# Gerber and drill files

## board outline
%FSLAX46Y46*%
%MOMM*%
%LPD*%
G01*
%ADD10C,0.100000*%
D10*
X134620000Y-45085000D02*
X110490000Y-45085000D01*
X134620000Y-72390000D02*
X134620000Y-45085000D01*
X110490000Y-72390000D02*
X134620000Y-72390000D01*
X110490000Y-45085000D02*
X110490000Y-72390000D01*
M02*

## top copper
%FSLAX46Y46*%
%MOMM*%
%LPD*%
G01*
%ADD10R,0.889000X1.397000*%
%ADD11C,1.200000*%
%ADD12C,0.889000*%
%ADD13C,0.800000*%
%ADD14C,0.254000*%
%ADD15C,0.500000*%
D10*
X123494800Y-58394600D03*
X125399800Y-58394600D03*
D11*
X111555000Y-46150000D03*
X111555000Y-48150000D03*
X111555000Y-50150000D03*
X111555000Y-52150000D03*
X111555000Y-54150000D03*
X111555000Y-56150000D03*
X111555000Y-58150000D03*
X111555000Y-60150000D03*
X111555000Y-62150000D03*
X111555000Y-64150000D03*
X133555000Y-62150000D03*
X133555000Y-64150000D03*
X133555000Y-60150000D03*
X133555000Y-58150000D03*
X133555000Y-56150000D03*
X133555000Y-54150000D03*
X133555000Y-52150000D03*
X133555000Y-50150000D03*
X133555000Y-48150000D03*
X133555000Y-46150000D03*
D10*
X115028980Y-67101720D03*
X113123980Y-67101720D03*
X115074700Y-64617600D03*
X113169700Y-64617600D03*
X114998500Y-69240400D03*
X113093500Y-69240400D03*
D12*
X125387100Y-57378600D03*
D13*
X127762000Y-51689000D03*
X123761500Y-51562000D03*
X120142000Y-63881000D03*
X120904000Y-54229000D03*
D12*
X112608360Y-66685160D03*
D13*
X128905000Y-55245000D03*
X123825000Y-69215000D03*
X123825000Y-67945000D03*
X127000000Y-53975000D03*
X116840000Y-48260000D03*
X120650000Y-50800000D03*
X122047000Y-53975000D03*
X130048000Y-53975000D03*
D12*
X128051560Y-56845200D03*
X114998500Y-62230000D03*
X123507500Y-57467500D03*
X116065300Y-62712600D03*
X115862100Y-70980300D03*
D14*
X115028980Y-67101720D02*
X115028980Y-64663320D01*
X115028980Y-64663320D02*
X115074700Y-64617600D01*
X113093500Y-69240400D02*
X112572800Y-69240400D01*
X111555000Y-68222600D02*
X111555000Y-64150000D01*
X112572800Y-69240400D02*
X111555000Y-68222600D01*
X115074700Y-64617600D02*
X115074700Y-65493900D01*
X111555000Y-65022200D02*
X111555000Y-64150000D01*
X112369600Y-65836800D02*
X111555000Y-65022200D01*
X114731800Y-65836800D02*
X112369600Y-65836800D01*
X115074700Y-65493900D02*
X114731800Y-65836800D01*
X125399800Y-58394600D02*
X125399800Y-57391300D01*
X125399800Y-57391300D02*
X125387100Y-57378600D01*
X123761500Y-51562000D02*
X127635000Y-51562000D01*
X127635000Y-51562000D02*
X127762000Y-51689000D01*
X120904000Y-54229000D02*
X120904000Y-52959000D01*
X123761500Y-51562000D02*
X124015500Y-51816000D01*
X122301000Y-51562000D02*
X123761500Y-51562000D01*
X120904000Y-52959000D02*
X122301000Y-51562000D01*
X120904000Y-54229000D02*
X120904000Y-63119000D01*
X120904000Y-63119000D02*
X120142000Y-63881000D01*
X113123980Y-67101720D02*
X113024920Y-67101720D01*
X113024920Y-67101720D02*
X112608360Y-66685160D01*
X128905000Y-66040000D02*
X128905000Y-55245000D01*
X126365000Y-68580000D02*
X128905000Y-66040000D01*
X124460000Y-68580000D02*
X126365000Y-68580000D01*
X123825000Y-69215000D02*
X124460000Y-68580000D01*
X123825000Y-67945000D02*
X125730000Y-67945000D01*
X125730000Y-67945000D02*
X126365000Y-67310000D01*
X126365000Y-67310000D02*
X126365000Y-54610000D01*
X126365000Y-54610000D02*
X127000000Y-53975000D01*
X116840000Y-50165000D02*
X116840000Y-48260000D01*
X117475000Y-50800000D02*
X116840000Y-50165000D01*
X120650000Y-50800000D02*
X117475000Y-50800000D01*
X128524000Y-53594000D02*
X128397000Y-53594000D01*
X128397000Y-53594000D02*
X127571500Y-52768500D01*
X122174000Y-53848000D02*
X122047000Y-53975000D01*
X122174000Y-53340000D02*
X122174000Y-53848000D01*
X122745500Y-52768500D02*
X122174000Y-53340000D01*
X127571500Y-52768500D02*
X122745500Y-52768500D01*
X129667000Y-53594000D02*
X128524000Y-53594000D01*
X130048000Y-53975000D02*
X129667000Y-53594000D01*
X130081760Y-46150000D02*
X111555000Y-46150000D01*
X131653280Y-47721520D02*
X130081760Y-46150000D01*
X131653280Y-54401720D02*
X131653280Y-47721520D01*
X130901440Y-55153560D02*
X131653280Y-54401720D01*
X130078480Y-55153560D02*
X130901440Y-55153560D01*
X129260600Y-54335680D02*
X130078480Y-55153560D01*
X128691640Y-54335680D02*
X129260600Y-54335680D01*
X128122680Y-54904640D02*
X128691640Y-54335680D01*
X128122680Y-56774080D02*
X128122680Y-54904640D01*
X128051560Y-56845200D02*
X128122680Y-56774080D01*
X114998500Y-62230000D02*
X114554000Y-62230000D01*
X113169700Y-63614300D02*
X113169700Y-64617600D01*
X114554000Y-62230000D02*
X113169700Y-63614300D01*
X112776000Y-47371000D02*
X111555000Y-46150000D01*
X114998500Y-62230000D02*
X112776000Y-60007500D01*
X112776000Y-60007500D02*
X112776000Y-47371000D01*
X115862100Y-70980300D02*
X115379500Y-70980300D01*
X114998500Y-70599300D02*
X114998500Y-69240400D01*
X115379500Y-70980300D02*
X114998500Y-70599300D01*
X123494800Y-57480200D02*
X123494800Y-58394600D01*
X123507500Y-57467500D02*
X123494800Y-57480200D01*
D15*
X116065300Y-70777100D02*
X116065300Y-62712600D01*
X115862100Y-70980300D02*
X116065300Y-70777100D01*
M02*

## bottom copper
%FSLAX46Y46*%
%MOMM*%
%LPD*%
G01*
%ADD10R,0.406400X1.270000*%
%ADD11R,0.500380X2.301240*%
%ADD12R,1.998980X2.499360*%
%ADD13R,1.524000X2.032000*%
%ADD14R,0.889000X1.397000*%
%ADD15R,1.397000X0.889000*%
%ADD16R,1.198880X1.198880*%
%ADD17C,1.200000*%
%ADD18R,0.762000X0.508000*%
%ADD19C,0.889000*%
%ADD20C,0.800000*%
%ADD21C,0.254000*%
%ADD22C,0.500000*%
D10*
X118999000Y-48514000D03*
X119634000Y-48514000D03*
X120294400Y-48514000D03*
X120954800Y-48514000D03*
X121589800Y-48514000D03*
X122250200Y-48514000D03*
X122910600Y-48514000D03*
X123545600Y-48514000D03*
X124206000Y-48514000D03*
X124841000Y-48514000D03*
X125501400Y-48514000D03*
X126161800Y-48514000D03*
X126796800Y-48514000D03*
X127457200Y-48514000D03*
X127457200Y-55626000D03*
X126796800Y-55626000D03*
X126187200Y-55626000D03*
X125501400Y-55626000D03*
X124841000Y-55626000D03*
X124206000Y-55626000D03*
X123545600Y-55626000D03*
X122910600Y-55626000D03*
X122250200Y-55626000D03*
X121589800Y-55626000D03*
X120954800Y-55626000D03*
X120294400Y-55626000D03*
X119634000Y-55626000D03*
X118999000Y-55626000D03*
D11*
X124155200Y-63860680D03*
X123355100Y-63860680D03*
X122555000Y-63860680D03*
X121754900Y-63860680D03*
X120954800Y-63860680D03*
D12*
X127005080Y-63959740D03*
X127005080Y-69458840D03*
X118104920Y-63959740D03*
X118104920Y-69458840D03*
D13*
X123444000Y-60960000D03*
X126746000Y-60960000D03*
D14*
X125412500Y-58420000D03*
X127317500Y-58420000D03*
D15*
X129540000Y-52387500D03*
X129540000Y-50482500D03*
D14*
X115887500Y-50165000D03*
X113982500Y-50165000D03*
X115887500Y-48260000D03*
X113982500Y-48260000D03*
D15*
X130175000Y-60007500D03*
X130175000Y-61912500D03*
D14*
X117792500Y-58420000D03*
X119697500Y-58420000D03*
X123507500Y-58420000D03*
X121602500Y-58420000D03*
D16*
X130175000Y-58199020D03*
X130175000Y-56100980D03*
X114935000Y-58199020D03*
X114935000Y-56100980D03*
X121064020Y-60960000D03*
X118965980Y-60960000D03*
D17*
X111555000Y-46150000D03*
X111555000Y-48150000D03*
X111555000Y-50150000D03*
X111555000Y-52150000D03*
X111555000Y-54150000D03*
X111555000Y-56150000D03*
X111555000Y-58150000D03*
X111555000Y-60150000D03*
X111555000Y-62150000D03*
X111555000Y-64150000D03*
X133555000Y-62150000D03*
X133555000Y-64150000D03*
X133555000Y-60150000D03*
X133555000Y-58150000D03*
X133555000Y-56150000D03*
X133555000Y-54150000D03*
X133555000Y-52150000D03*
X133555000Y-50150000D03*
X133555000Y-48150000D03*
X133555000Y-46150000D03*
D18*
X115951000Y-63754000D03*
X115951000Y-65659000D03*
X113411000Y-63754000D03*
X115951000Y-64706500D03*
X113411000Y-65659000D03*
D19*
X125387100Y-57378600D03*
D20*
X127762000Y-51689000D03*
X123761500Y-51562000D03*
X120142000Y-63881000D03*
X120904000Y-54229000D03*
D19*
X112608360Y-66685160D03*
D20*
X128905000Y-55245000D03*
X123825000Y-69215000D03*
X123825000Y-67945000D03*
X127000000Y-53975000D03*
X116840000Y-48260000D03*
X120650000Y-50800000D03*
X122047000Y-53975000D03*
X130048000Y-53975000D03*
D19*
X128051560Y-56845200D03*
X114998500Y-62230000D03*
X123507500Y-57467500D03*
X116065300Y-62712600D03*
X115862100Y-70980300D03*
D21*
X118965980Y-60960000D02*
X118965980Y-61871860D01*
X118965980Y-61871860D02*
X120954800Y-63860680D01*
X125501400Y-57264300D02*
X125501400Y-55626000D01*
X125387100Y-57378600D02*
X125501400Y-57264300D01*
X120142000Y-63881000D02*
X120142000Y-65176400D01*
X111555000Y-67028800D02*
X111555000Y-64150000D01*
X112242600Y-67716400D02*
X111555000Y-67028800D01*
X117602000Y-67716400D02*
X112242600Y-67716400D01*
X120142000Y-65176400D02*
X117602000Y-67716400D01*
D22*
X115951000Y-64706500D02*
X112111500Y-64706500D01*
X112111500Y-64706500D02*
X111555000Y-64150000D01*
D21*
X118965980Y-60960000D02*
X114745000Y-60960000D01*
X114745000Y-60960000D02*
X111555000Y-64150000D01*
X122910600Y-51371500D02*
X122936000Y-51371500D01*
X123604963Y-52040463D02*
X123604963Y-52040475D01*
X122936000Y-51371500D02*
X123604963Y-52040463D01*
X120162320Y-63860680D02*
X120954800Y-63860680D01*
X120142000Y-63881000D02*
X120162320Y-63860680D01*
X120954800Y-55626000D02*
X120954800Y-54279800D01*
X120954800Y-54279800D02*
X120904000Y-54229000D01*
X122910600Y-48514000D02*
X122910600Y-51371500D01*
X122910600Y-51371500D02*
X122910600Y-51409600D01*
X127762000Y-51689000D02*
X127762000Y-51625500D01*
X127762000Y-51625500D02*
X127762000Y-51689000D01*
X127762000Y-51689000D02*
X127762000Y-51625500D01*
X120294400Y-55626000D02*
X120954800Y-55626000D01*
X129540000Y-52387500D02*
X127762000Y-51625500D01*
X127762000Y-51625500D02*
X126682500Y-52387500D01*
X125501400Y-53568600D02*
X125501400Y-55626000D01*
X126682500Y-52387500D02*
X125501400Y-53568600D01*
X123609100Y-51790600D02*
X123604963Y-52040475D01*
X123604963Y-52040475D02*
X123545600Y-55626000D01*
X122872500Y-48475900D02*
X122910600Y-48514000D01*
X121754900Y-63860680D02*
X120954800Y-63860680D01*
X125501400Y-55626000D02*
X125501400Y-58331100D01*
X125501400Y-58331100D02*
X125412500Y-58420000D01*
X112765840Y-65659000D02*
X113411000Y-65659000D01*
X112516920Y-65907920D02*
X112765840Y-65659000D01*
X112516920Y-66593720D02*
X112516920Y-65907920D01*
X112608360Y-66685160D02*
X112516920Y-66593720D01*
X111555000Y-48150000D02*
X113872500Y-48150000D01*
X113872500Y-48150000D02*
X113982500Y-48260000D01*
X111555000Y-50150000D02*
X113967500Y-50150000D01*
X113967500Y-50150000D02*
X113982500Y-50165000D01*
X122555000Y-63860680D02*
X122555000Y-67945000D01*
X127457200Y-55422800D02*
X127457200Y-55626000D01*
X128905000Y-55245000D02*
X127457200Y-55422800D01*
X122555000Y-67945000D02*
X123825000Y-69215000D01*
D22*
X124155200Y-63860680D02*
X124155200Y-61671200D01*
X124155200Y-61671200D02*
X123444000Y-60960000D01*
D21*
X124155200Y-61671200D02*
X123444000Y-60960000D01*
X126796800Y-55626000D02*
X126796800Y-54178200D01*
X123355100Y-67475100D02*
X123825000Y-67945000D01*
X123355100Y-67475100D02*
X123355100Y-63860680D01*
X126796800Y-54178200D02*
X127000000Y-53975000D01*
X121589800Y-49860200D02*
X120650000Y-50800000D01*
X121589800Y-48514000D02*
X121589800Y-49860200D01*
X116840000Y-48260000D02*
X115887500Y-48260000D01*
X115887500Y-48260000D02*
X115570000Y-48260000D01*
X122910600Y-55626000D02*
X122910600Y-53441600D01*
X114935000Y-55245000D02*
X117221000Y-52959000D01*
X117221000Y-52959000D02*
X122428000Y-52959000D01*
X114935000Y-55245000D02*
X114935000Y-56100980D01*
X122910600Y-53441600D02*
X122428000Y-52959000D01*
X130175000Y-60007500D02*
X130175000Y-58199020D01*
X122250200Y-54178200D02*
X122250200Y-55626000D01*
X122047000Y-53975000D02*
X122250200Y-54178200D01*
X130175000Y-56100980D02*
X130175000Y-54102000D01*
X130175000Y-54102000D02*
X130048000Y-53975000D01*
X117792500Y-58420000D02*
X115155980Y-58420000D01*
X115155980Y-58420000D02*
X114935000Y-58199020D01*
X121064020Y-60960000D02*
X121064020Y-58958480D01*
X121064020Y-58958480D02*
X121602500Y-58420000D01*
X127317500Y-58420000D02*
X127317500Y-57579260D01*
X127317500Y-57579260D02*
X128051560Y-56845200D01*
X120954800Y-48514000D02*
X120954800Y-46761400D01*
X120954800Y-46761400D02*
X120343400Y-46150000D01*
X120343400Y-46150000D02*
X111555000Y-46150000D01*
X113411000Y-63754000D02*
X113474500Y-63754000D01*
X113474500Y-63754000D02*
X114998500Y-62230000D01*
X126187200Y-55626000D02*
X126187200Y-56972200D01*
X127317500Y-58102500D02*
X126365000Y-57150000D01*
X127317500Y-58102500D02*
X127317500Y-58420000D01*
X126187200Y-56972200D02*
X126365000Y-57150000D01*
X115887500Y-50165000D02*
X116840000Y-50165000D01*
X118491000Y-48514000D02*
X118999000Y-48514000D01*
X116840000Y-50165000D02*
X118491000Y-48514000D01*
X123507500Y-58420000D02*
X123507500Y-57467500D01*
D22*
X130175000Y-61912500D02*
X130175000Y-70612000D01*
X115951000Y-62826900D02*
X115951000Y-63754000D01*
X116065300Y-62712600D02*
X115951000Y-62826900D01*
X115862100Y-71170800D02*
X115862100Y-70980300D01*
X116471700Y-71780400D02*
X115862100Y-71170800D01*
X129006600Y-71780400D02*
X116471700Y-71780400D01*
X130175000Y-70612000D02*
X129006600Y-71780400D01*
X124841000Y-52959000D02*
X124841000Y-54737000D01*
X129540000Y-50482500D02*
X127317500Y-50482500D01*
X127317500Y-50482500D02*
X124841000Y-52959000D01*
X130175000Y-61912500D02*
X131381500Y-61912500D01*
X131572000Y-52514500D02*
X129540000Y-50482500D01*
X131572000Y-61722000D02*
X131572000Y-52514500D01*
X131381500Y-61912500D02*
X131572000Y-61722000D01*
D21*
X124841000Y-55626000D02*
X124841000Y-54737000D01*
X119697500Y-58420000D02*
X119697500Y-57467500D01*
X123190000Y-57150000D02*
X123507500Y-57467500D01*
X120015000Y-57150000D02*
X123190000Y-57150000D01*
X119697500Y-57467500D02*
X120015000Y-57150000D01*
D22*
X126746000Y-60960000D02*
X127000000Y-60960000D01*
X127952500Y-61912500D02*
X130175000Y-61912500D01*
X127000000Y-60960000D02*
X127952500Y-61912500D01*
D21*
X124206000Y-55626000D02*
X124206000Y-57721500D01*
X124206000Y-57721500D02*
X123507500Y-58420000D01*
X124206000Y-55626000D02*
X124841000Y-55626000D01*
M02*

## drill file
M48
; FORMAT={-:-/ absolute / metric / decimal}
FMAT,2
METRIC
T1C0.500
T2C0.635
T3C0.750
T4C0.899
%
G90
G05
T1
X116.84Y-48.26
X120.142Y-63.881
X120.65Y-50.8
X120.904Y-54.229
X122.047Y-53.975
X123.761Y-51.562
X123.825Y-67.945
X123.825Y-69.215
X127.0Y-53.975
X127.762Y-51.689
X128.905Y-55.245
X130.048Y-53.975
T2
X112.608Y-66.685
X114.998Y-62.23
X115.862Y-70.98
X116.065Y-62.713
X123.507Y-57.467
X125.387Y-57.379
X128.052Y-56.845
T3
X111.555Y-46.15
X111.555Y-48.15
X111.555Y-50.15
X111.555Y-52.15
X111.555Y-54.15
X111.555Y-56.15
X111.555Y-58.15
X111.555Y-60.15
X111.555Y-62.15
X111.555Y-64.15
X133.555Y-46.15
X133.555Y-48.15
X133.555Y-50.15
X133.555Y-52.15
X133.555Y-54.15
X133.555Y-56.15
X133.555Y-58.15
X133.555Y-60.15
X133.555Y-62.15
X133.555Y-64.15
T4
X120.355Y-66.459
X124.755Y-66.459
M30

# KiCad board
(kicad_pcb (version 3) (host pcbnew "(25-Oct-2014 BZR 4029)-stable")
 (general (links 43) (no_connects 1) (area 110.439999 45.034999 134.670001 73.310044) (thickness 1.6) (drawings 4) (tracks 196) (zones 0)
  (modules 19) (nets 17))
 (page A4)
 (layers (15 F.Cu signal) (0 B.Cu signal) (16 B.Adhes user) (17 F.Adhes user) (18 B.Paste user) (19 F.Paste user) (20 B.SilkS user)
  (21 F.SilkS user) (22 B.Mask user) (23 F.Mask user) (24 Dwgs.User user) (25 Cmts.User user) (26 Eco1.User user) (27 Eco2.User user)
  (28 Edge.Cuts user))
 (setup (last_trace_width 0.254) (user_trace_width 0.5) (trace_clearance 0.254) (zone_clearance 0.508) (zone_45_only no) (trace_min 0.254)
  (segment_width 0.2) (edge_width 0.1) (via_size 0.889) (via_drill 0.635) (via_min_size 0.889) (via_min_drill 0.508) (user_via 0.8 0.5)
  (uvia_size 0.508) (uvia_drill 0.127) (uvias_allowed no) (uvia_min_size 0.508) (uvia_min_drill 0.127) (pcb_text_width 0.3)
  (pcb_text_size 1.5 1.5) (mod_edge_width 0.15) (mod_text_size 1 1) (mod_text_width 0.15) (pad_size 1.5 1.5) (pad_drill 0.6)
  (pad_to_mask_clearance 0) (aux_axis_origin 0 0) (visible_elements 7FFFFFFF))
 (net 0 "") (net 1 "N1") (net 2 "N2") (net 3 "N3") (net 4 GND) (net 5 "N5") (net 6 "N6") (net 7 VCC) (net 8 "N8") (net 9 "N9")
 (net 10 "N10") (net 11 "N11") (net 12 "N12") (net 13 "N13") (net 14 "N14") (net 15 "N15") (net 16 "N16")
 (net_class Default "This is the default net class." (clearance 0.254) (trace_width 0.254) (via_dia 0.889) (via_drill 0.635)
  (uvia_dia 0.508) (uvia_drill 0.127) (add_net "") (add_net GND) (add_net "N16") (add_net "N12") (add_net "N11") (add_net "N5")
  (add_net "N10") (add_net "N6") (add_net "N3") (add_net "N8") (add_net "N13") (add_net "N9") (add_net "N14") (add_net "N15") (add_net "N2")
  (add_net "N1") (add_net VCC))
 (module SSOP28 (layer B.Cu) (at 123.19 52.07)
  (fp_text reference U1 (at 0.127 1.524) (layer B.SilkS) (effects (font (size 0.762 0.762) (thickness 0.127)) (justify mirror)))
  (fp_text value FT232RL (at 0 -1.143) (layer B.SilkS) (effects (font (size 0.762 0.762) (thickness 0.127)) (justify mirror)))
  (pad 1 smd rect (at -4.191 -3.556) (size 0.4064 1.27) (layers B.Cu B.Paste B.Mask) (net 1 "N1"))
  (pad 2 smd rect (at -3.556 -3.556) (size 0.4064 1.27) (layers B.Cu B.Paste B.Mask))
  (pad 3 smd rect (at -2.8956 -3.556) (size 0.4064 1.27) (layers B.Cu B.Paste B.Mask))
  (pad 4 smd rect (at -2.2352 -3.556) (size 0.4064 1.27) (layers B.Cu B.Paste B.Mask) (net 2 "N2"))
  (pad 5 smd rect (at -1.6002 -3.556) (size 0.4064 1.27) (layers B.Cu B.Paste B.Mask) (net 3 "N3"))
  (pad 6 smd rect (at -0.9398 -3.556) (size 0.4064 1.27) (layers B.Cu B.Paste B.Mask))
  (pad 7 smd rect (at -0.2794 -3.556) (size 0.4064 1.27) (layers B.Cu B.Paste B.Mask) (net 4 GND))
  (pad 8 smd rect (at 0.3556 -3.556) (size 0.4064 1.27) (layers B.Cu B.Paste B.Mask))
  (pad 9 smd rect (at 1.016 -3.556) (size 0.4064 1.27) (layers B.Cu B.Paste B.Mask))
  (pad 10 smd rect (at 1.651 -3.556) (size 0.4064 1.27) (layers B.Cu B.Paste B.Mask))
  (pad 11 smd rect (at 2.3114 -3.556) (size 0.4064 1.27) (layers B.Cu B.Paste B.Mask))
  (pad 12 smd rect (at 2.9718 -3.556) (size 0.4064 1.27) (layers B.Cu B.Paste B.Mask))
  (pad 13 smd rect (at 3.6068 -3.556) (size 0.4064 1.27) (layers B.Cu B.Paste B.Mask))
  (pad 14 smd rect (at 4.2672 -3.556) (size 0.4064 1.27) (layers B.Cu B.Paste B.Mask))
  (pad 15 smd rect (at 4.2672 3.556) (size 0.4064 1.27) (layers B.Cu B.Paste B.Mask) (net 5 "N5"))
  (pad 16 smd rect (at 3.6068 3.556) (size 0.4064 1.27) (layers B.Cu B.Paste B.Mask) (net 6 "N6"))
  (pad 17 smd rect (at 2.9972 3.556) (size 0.4064 1.27) (layers B.Cu B.Paste B.Mask) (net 2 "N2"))
  (pad 18 smd rect (at 2.3114 3.556) (size 0.4064 1.27) (layers B.Cu B.Paste B.Mask) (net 4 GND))
  (pad 19 smd rect (at 1.651 3.556) (size 0.4064 1.27) (layers B.Cu B.Paste B.Mask) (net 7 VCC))
  (pad 20 smd rect (at 1.016 3.556) (size 0.4064 1.27) (layers B.Cu B.Paste B.Mask) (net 7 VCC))
  (pad 21 smd rect (at 0.3556 3.556) (size 0.4064 1.27) (layers B.Cu B.Paste B.Mask) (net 4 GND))
  (pad 22 smd rect (at -0.2794 3.556) (size 0.4064 1.27) (layers B.Cu B.Paste B.Mask) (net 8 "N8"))
  (pad 23 smd rect (at -0.9398 3.556) (size 0.4064 1.27) (layers B.Cu B.Paste B.Mask) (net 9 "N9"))
  (pad 24 smd rect (at -1.6002 3.556) (size 0.4064 1.27) (layers B.Cu B.Paste B.Mask))
  (pad 25 smd rect (at -2.2352 3.556) (size 0.4064 1.27) (layers B.Cu B.Paste B.Mask) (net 4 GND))
  (pad 26 smd rect (at -2.8956 3.556) (size 0.4064 1.27) (layers B.Cu B.Paste B.Mask) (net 4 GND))
  (pad 27 smd rect (at -3.556 3.556) (size 0.4064 1.27) (layers B.Cu B.Paste B.Mask))
  (pad 28 smd rect (at -4.191 3.556) (size 0.4064 1.27) (layers B.Cu B.Paste B.Mask)))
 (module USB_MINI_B (layer B.Cu) (at 122.555 67.31 90)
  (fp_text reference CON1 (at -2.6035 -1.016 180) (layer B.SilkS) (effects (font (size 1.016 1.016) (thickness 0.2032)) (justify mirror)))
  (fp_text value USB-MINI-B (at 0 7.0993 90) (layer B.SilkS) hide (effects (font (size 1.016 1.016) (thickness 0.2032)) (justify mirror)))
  (pad 1 smd rect (at 3.44932 1.6002 90) (size 2.30124 0.50038) (layers B.Cu B.Paste B.Mask) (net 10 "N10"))
  (pad 2 smd rect (at 3.44932 0.8001 90) (size 2.30124 0.50038) (layers B.Cu B.Paste B.Mask) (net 6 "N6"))
  (pad 3 smd rect (at 3.44932 0 90) (size 2.30124 0.50038) (layers B.Cu B.Paste B.Mask) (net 5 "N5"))
  (pad 4 smd rect (at 3.44932 -0.8001 90) (size 2.30124 0.50038) (layers B.Cu B.Paste B.Mask) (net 4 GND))
  (pad 5 smd rect (at 3.44932 -1.6002 90) (size 2.30124 0.50038) (layers B.Cu B.Paste B.Mask) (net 4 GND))
  (pad 6 smd rect (at 3.35026 4.45008 90) (size 2.49936 1.99898) (layers B.Cu B.Paste B.Mask))
  (pad 7 smd rect (at -2.14884 4.45008 90) (size 2.49936 1.99898) (layers B.Cu B.Paste B.Mask))
  (pad 8 smd rect (at 3.35026 -4.45008 90) (size 2.49936 1.99898) (layers B.Cu B.Paste B.Mask))
  (pad 9 smd rect (at -2.14884 -4.45008 90) (size 2.49936 1.99898) (layers B.Cu B.Paste B.Mask))
  (pad "" np_thru_hole circle (at 0.8509 2.19964 90) (size 0.89916 0.89916) (drill 0.89916) (layers *.Cu *.Mask B.SilkS))
  (pad 2 np_thru_hole circle (at 0.8509 -2.19964 90) (size 0.89916 0.89916) (drill 0.89916) (layers *.Cu *.Mask B.SilkS) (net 6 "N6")))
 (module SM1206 (layer B.Cu) (at 125.095 60.96)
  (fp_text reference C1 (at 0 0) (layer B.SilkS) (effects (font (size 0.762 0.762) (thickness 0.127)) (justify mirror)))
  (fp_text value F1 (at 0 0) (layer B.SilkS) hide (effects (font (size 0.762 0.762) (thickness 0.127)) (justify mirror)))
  (pad 1 smd rect (at -1.651 0) (size 1.524 2.032) (layers B.Cu B.Paste B.Mask) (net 10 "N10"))
  (pad 2 smd rect (at 1.651 0) (size 1.524 2.032) (layers B.Cu B.Paste B.Mask) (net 7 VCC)))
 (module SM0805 (layer F.Cu) (at 124.4473 58.3946)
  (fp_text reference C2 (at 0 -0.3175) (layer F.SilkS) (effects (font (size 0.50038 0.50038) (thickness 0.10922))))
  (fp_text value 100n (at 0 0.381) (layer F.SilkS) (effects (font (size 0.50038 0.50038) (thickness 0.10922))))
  (pad 1 smd rect (at -0.9525 0) (size 0.889 1.397) (layers F.Cu F.Paste F.Mask) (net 7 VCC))
  (pad 2 smd rect (at 0.9525 0) (size 0.889 1.397) (layers F.Cu F.Paste F.Mask) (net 4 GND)))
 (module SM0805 (layer B.Cu) (at 126.365 58.42)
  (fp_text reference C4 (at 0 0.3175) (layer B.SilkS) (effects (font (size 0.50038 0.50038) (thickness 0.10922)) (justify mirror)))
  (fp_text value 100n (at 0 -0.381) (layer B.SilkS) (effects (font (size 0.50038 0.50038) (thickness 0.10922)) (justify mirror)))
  (pad 1 smd rect (at -0.9525 0) (size 0.889 1.397) (layers B.Cu B.Paste B.Mask) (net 4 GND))
  (pad 2 smd rect (at 0.9525 0) (size 0.889 1.397) (layers B.Cu B.Paste B.Mask) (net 2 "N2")))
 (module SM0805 (layer B.Cu) (at 129.54 51.435 90)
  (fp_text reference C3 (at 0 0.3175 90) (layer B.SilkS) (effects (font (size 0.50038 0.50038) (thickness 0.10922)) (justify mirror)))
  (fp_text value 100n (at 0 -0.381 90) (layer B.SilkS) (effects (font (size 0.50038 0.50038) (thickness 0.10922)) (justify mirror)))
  (pad 1 smd rect (at -0.9525 0 90) (size 0.889 1.397) (layers B.Cu B.Paste B.Mask) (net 4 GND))
  (pad 2 smd rect (at 0.9525 0 90) (size 0.889 1.397) (layers B.Cu B.Paste B.Mask) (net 7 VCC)))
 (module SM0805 (layer B.Cu) (at 114.935 50.165 180)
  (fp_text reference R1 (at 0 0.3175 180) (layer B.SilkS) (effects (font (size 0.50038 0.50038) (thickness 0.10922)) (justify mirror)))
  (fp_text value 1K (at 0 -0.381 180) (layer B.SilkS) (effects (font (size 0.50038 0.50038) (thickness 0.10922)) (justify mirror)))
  (pad 1 smd rect (at -0.9525 0 180) (size 0.889 1.397) (layers B.Cu B.Paste B.Mask) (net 1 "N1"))
  (pad 2 smd rect (at 0.9525 0 180) (size 0.889 1.397) (layers B.Cu B.Paste B.Mask) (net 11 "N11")))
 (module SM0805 (layer B.Cu) (at 114.935 48.26 180)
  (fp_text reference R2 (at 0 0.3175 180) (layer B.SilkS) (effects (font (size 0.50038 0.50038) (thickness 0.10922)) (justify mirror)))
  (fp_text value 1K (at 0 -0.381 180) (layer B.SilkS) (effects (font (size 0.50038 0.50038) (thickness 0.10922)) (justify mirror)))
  (pad 1 smd rect (at -0.9525 0 180) (size 0.889 1.397) (layers B.Cu B.Paste B.Mask) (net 3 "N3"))
  (pad 2 smd rect (at 0.9525 0 180) (size 0.889 1.397) (layers B.Cu B.Paste B.Mask) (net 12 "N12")))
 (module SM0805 (layer B.Cu) (at 130.175 60.96 270)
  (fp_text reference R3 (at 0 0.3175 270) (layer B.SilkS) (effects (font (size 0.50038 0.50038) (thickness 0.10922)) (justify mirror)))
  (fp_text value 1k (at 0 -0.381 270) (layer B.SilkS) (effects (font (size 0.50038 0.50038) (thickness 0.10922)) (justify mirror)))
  (pad 1 smd rect (at -0.9525 0 270) (size 0.889 1.397) (layers B.Cu B.Paste B.Mask) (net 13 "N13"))
  (pad 2 smd rect (at 0.9525 0 270) (size 0.889 1.397) (layers B.Cu B.Paste B.Mask) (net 7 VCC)))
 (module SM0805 (layer B.Cu) (at 118.745 58.42)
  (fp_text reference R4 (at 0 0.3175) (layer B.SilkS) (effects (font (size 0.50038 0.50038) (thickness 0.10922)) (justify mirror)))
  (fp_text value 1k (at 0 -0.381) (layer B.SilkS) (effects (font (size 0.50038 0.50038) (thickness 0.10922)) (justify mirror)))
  (pad 1 smd rect (at -0.9525 0) (size 0.889 1.397) (layers B.Cu B.Paste B.Mask) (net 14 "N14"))
  (pad 2 smd rect (at 0.9525 0) (size 0.889 1.397) (layers B.Cu B.Paste B.Mask) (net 7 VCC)))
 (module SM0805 (layer B.Cu) (at 122.555 58.42 180)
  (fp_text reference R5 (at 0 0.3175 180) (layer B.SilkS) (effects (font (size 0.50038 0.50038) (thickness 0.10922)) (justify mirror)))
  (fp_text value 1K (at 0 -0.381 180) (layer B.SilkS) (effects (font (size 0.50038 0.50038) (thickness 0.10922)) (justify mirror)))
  (pad 1 smd rect (at -0.9525 0 180) (size 0.889 1.397) (layers B.Cu B.Paste B.Mask) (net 7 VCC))
  (pad 2 smd rect (at 0.9525 0 180) (size 0.889 1.397) (layers B.Cu B.Paste B.Mask) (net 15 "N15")))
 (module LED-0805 (layer B.Cu) (at 130.175 57.15 90)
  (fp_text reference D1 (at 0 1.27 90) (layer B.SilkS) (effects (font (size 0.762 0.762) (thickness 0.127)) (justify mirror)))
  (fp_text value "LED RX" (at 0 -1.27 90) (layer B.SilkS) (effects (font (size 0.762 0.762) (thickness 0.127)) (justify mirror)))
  (pad 1 smd rect (at -1.04902 0 90) (size 1.19888 1.19888) (layers B.Cu B.Paste B.Mask) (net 13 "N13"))
  (pad 2 smd rect (at 1.04902 0 90) (size 1.19888 1.19888) (layers B.Cu B.Paste B.Mask) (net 9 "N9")))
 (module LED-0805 (layer B.Cu) (at 114.935 57.15 90)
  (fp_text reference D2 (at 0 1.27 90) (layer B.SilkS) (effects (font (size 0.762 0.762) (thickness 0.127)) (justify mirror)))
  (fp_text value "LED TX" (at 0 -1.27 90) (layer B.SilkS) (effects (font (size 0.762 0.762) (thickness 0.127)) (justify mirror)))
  (pad 1 smd rect (at -1.04902 0 90) (size 1.19888 1.19888) (layers B.Cu B.Paste B.Mask) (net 14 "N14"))
  (pad 2 smd rect (at 1.04902 0 90) (size 1.19888 1.19888) (layers B.Cu B.Paste B.Mask) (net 8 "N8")))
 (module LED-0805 (layer B.Cu) (at 120.015 60.96 180)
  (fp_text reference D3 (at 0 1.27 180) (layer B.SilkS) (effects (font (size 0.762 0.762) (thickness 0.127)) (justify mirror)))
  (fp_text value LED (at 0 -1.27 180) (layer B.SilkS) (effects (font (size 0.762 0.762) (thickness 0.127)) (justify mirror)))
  (pad 1 smd rect (at -1.04902 0 180) (size 1.19888 1.19888) (layers B.Cu B.Paste B.Mask) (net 15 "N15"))
  (pad 2 smd rect (at 1.04902 0 180) (size 1.19888 1.19888) (layers B.Cu B.Paste B.Mask) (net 4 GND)))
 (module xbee (layer F.Cu) (at 122.555 57.15)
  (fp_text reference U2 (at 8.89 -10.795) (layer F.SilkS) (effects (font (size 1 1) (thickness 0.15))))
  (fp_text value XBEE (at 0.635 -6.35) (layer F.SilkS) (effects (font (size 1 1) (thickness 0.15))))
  (pad 1 thru_hole circle (at -11 -11) (size 1.2 1.2) (drill 0.75) (layers *.Cu *.Mask F.SilkS) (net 2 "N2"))
  (pad 2 thru_hole circle (at -11 -9) (size 1.2 1.2) (drill 0.75) (layers *.Cu *.Mask F.SilkS) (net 12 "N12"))
  (pad 3 thru_hole circle (at -11 -7) (size 1.2 1.2) (drill 0.75) (layers *.Cu *.Mask F.SilkS) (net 11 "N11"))
  (pad 4 thru_hole circle (at -11 -5) (size 1.2 1.2) (drill 0.75) (layers *.Cu *.Mask F.SilkS))
  (pad 5 thru_hole circle (at -11 -3) (size 1.2 1.2) (drill 0.75) (layers *.Cu *.Mask F.SilkS))
  (pad 6 thru_hole circle (at -11 -1) (size 1.2 1.2) (drill 0.75) (layers *.Cu *.Mask F.SilkS))
  (pad 7 thru_hole circle (at -11 1) (size 1.2 1.2) (drill 0.75) (layers *.Cu *.Mask F.SilkS))
  (pad 8 thru_hole circle (at -11 3) (size 1.2 1.2) (drill 0.75) (layers *.Cu *.Mask F.SilkS))
  (pad 9 thru_hole circle (at -11 5) (size 1.2 1.2) (drill 0.75) (layers *.Cu *.Mask F.SilkS))
  (pad 10 thru_hole circle (at -11 7) (size 1.2 1.2) (drill 0.75) (layers *.Cu *.Mask F.SilkS) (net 4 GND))
  (pad 12 thru_hole circle (at 11 5) (size 1.2 1.2) (drill 0.75) (layers *.Cu *.Mask F.SilkS))
  (pad 11 thru_hole circle (at 11 7) (size 1.2 1.2) (drill 0.75) (layers *.Cu *.Mask F.SilkS))
  (pad 13 thru_hole circle (at 11 3) (size 1.2 1.2) (drill 0.75) (layers *.Cu *.Mask F.SilkS))
  (pad 14 thru_hole circle (at 11 1) (size 1.2 1.2) (drill 0.75) (layers *.Cu *.Mask F.SilkS))
  (pad 15 thru_hole circle (at 11 -1) (size 1.2 1.2) (drill 0.75) (layers *.Cu *.Mask F.SilkS))
  (pad 16 thru_hole circle (at 11 -3) (size 1.2 1.2) (drill 0.75) (layers *.Cu *.Mask F.SilkS))
  (pad 17 thru_hole circle (at 11 -5) (size 1.2 1.2) (drill 0.75) (layers *.Cu *.Mask F.SilkS))
  (pad 18 thru_hole circle (at 11 -7) (size 1.2 1.2) (drill 0.75) (layers *.Cu *.Mask F.SilkS))
  (pad 19 thru_hole circle (at 11 -9) (size 1.2 1.2) (drill 0.75) (layers *.Cu *.Mask F.SilkS))
  (pad 20 thru_hole circle (at 11 -11) (size 1.2 1.2) (drill 0.75) (layers *.Cu *.Mask F.SilkS)))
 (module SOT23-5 (layer B.Cu) (at 114.681 64.7065 270)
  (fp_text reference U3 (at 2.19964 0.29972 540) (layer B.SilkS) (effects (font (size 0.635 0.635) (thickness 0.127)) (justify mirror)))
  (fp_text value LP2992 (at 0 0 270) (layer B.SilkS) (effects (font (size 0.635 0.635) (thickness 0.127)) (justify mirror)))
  (pad 1 smd rect (at -0.9525 -1.27 270) (size 0.508 0.762) (layers B.Cu B.Paste B.Mask) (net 7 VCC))
  (pad 3 smd rect (at 0.9525 -1.27 270) (size 0.508 0.762) (layers B.Cu B.Paste B.Mask))
  (pad 5 smd rect (at -0.9525 1.27 270) (size 0.508 0.762) (layers B.Cu B.Paste B.Mask) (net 2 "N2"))
  (pad 2 smd rect (at 0 -1.27 270) (size 0.508 0.762) (layers B.Cu B.Paste B.Mask) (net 4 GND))
  (pad 4 smd rect (at 0.9525 1.27 270) (size 0.508 0.762) (layers B.Cu B.Paste B.Mask) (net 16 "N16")))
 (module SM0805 (layer F.Cu) (at 114.07648 67.10172 180)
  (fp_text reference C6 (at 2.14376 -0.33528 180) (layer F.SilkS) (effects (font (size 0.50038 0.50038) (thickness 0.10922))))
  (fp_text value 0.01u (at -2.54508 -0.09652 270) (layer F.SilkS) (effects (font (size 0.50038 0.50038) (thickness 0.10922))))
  (pad 1 smd rect (at -0.9525 0 180) (size 0.889 1.397) (layers F.Cu F.Paste F.Mask) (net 4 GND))
  (pad 2 smd rect (at 0.9525 0 180) (size 0.889 1.397) (layers F.Cu F.Paste F.Mask) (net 16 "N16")))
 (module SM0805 (layer F.Cu) (at 114.1222 64.6176 180)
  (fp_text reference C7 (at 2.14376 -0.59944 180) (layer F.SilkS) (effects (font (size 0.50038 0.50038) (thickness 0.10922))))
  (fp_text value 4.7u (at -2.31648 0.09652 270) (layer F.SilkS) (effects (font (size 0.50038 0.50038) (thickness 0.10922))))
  (pad 1 smd rect (at -0.9525 0 180) (size 0.889 1.397) (layers F.Cu F.Paste F.Mask) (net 4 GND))
  (pad 2 smd rect (at 0.9525 0 180) (size 0.889 1.397) (layers F.Cu F.Paste F.Mask) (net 2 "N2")))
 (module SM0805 (layer F.Cu) (at 114.046 69.2404 180)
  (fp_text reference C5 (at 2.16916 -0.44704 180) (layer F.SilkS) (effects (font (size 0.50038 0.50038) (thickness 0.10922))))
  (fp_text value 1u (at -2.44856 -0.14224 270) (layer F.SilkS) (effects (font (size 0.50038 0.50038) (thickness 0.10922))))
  (pad 1 smd rect (at -0.9525 0 180) (size 0.889 1.397) (layers F.Cu F.Paste F.Mask) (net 7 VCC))
  (pad 2 smd rect (at 0.9525 0 180) (size 0.889 1.397) (layers F.Cu F.Paste F.Mask) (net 4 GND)))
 (gr_line (start 134.62 45.085) (end 110.49 45.085) (angle 90) (layer Edge.Cuts) (width 0.1))
 (gr_line (start 134.62 72.39) (end 134.62 45.085) (angle 90) (layer Edge.Cuts) (width 0.1))
 (gr_line (start 110.49 72.39) (end 134.62 72.39) (angle 90) (layer Edge.Cuts) (width 0.1))
 (gr_line (start 110.49 45.085) (end 110.49 72.39) (angle 90) (layer Edge.Cuts) (width 0.1))
 (segment (start 118.96598 60.96) (end 118.96598 61.87186) (width 0.254) (layer B.Cu) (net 4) (status 400000))
 (segment (start 118.96598 61.87186) (end 120.9548 63.86068) (width 0.254) (layer B.Cu) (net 4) (status 800000))
 (segment (start 115.02898 67.10172) (end 115.02898 64.66332) (width 0.254) (layer F.Cu) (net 4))
 (segment (start 115.02898 64.66332) (end 115.0747 64.6176) (width 0.254) (layer F.Cu) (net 4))
 (segment (start 113.0935 69.2404) (end 112.5728 69.2404) (width 0.254) (layer F.Cu) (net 4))
 (segment (start 111.555 68.2226) (end 111.555 64.15) (width 0.254) (layer F.Cu) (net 4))
 (segment (start 112.5728 69.2404) (end 111.555 68.2226) (width 0.254) (layer F.Cu) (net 4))
 (segment (start 115.0747 64.6176) (end 115.0747 65.4939) (width 0.254) (layer F.Cu) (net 4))
 (segment (start 111.555 65.0222) (end 111.555 64.15) (width 0.254) (layer F.Cu) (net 4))
 (segment (start 112.3696 65.8368) (end 111.555 65.0222) (width 0.254) (layer F.Cu) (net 4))
 (segment (start 114.7318 65.8368) (end 112.3696 65.8368) (width 0.254) (layer F.Cu) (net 4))
 (segment (start 115.0747 65.4939) (end 114.7318 65.8368) (width 0.254) (layer F.Cu) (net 4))
 (segment (start 125.3998 58.3946) (end 125.3998 57.3913) (width 0.254) (layer F.Cu) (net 4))
 (segment (start 125.5014 57.2643) (end 125.5014 55.626) (width 0.254) (layer B.Cu) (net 4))
 (segment (start 125.3871 57.3786) (end 125.5014 57.2643) (width 0.254) (layer B.Cu) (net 4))
 (via (at 125.3871 57.3786) (size 0.889) (layers F.Cu B.Cu) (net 4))
 (segment (start 125.3998 57.3913) (end 125.3871 57.3786) (width 0.254) (layer F.Cu) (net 4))
 (segment (start 120.142 63.881) (end 120.142 65.1764) (width 0.254) (layer B.Cu) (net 4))
 (segment (start 111.555 67.0288) (end 111.555 64.15) (width 0.254) (layer B.Cu) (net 4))
 (segment (start 112.2426 67.7164) (end 111.555 67.0288) (width 0.254) (layer B.Cu) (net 4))
 (segment (start 117.602 67.7164) (end 112.2426 67.7164) (width 0.254) (layer B.Cu) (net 4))
 (segment (start 120.142 65.1764) (end 117.602 67.7164) (width 0.254) (layer B.Cu) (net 4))
 (segment (start 115.951 64.7065) (end 112.1115 64.7065) (width 0.5) (layer B.Cu) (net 4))
 (segment (start 112.1115 64.7065) (end 111.555 64.15) (width 0.5) (layer B.Cu) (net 4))
 (segment (start 118.96598 60.96) (end 114.745 60.96) (width 0.254) (layer B.Cu) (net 4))
 (segment (start 114.745 60.96) (end 111.555 64.15) (width 0.254) (layer B.Cu) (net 4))
 (segment (start 123.7615 51.562) (end 127.635 51.562) (width 0.254) (layer F.Cu) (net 4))
 (via (at 127.762 51.689) (size 0.8) (drill 0.5) (layers F.Cu B.Cu) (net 4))
 (via (at 123.7615 51.562) (size 0.8) (drill 0.5) (layers F.Cu B.Cu) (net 4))
 (segment (start 127.635 51.562) (end 127.762 51.689) (width 0.254) (layer F.Cu) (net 4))
 (segment (start 120.904 54.229) (end 120.904 52.959) (width 0.254) (layer F.Cu) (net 4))
 (segment (start 123.7615 51.562) (end 124.0155 51.816) (width 0.254) (layer F.Cu) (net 4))
 (segment (start 122.301 51.562) (end 123.7615 51.562) (width 0.254) (layer F.Cu) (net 4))
 (segment (start 120.904 52.959) (end 122.301 51.562) (width 0.254) (layer F.Cu) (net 4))
 (segment (start 122.9106 51.3715) (end 122.936 51.3715) (width 0.254) (layer B.Cu) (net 4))
 (segment (start 123.604963 52.040463) (end 123.604963 52.040475) (width 0.254) (layer B.Cu) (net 4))
 (segment (start 122.936 51.3715) (end 123.604963 52.040463) (width 0.254) (layer B.Cu) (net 4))
 (segment (start 120.904 54.229) (end 120.904 63.119) (width 0.254) (layer F.Cu) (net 4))
 (segment (start 120.16232 63.86068) (end 120.9548 63.86068) (width 0.254) (layer B.Cu) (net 4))
 (segment (start 120.142 63.881) (end 120.16232 63.86068) (width 0.254) (layer B.Cu) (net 4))
 (via (at 120.142 63.881) (size 0.8) (drill 0.5) (layers F.Cu B.Cu) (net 4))
 (segment (start 120.904 63.119) (end 120.142 63.881) (width 0.254) (layer F.Cu) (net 4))
 (segment (start 120.9548 55.626) (end 120.9548 54.2798) (width 0.254) (layer B.Cu) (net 4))
 (via (at 120.904 54.229) (size 0.8) (drill 0.5) (layers F.Cu B.Cu) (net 4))
 (segment (start 120.9548 54.2798) (end 120.904 54.229) (width 0.254) (layer B.Cu) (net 4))
 (segment (start 122.9106 48.514) (end 122.9106 51.3715) (width 0.254) (layer B.Cu) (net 4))
 (segment (start 122.9106 51.3715) (end 122.9106 51.4096) (width 0.254) (layer B.Cu) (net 4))
 (segment (start 127.762 51.689) (end 127.762 51.6255) (width 0.254) (layer B.Cu) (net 4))
 (segment (start 127.762 51.6255) (end 127.762 51.689) (width 0.254) (layer B.Cu) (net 4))
 (segment (start 127.762 51.689) (end 127.762 51.6255) (width 0.254) (layer B.Cu) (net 4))
 (segment (start 120.2944 55.626) (end 120.9548 55.626) (width 0.254) (layer B.Cu) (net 4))
 (segment (start 129.54 52.3875) (end 127.762 51.6255) (width 0.254) (layer B.Cu) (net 4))
 (segment (start 127.762 51.6255) (end 126.6825 52.3875) (width 0.254) (layer B.Cu) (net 4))
 (segment (start 125.5014 53.5686) (end 125.5014 55.626) (width 0.254) (layer B.Cu) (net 4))
 (segment (start 126.6825 52.3875) (end 125.5014 53.5686) (width 0.254) (layer B.Cu) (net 4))
 (segment (start 123.6091 51.7906) (end 123.604963 52.040475) (width 0.254) (layer B.Cu) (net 4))
 (segment (start 123.604963 52.040475) (end 123.5456 55.626) (width 0.254) (layer B.Cu) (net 4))
 (segment (start 122.8725 48.4759) (end 122.9106 48.514) (width 0.254) (layer B.Cu) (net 4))
 (segment (start 121.7549 63.86068) (end 120.9548 63.86068) (width 0.254) (layer B.Cu) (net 4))
 (segment (start 125.5014 55.626) (end 125.5014 58.3311) (width 0.254) (layer B.Cu) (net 4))
 (segment (start 125.5014 58.3311) (end 125.4125 58.42) (width 0.254) (layer B.Cu) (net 4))
 (segment (start 113.12398 67.10172) (end 113.02492 67.10172) (width 0.254) (layer F.Cu) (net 16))
 (segment (start 112.76584 65.659) (end 113.411 65.659) (width 0.254) (layer B.Cu) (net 16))
 (segment (start 112.51692 65.90792) (end 112.76584 65.659) (width 0.254) (layer B.Cu) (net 16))
 (segment (start 112.51692 66.59372) (end 112.51692 65.90792) (width 0.254) (layer B.Cu) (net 16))
 (segment (start 112.60836 66.68516) (end 112.51692 66.59372) (width 0.254) (layer B.Cu) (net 16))
 (via (at 112.60836 66.68516) (size 0.889) (layers F.Cu B.Cu) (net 16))
 (segment (start 113.02492 67.10172) (end 112.60836 66.68516) (width 0.254) (layer F.Cu) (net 16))
 (segment (start 111.555 48.15) (end 113.8725 48.15) (width 0.254) (layer B.Cu) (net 12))
 (segment (start 113.8725 48.15) (end 113.9825 48.26) (width 0.254) (layer B.Cu) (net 12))
 (segment (start 111.555 50.15) (end 113.9675 50.15) (width 0.254) (layer B.Cu) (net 11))
 (segment (start 113.9675 50.15) (end 113.9825 50.165) (width 0.254) (layer B.Cu) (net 11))
 (segment (start 122.555 63.86068) (end 122.555 67.945) (width 0.254) (layer B.Cu) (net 5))
 (segment (start 127.4572 55.4228) (end 127.4572 55.626) (width 0.254) (layer B.Cu) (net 5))
 (segment (start 128.905 55.245) (end 127.4572 55.4228) (width 0.254) (layer B.Cu) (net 5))
 (via (at 128.905 55.245) (size 0.8) (drill 0.5) (layers F.Cu B.Cu) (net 5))
 (segment (start 128.905 66.04) (end 128.905 55.245) (width 0.254) (layer F.Cu) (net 5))
 (segment (start 126.365 68.58) (end 128.905 66.04) (width 0.254) (layer F.Cu) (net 5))
 (segment (start 124.46 68.58) (end 126.365 68.58) (width 0.254) (layer F.Cu) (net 5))
 (segment (start 123.825 69.215) (end 124.46 68.58) (width 0.254) (layer F.Cu) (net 5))
 (via (at 123.825 69.215) (size 0.8) (drill 0.5) (layers F.Cu B.Cu) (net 5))
 (segment (start 122.555 67.945) (end 123.825 69.215) (width 0.254) (layer B.Cu) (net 5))
 (segment (start 124.1552 63.86068) (end 124.1552 61.6712) (width 0.5) (layer B.Cu) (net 10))
 (segment (start 124.1552 61.6712) (end 123.444 60.96) (width 0.5) (layer B.Cu) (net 10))
 (segment (start 124.1552 61.6712) (end 123.444 60.96) (width 0.254) (layer B.Cu) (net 10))
 (segment (start 126.7968 55.626) (end 126.7968 54.1782) (width 0.254) (layer B.Cu) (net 6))
 (segment (start 123.3551 67.4751) (end 123.825 67.945) (width 0.254) (layer B.Cu) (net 6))
 (via (at 123.825 67.945) (size 0.8) (drill 0.5) (layers F.Cu B.Cu) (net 6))
 (segment (start 123.825 67.945) (end 125.73 67.945) (width 0.254) (layer F.Cu) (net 6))
 (segment (start 125.73 67.945) (end 126.365 67.31) (width 0.254) (layer F.Cu) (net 6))
 (segment (start 126.365 67.31) (end 126.365 54.61) (width 0.254) (layer F.Cu) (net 6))
 (segment (start 126.365 54.61) (end 127 53.975) (width 0.254) (layer F.Cu) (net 6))
 (segment (start 123.3551 67.4751) (end 123.3551 63.86068) (width 0.254) (layer B.Cu) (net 6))
 (via (at 127 53.975) (size 0.8) (drill 0.5) (layers F.Cu B.Cu) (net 6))
 (segment (start 126.7968 54.1782) (end 127 53.975) (width 0.254) (layer B.Cu) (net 6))
 (segment (start 121.5898 49.8602) (end 120.65 50.8) (width 0.254) (layer B.Cu) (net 3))
 (segment (start 121.5898 48.514) (end 121.5898 49.8602) (width 0.254) (layer B.Cu) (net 3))
 (segment (start 116.84 48.26) (end 115.8875 48.26) (width 0.254) (layer B.Cu) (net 3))
 (via (at 116.84 48.26) (size 0.8) (drill 0.5) (layers F.Cu B.Cu) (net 3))
 (segment (start 116.84 50.165) (end 116.84 48.26) (width 0.254) (layer F.Cu) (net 3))
 (segment (start 117.475 50.8) (end 116.84 50.165) (width 0.254) (layer F.Cu) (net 3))
 (segment (start 120.65 50.8) (end 117.475 50.8) (width 0.254) (layer F.Cu) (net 3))
 (via (at 120.65 50.8) (size 0.8) (drill 0.5) (layers F.Cu B.Cu) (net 3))
 (segment (start 115.8875 48.26) (end 115.57 48.26) (width 0.254) (layer B.Cu) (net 3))
 (segment (start 122.9106 55.626) (end 122.9106 53.4416) (width 0.254) (layer B.Cu) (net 8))
 (segment (start 114.935 55.245) (end 117.221 52.959) (width 0.254) (layer B.Cu) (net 8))
 (segment (start 117.221 52.959) (end 122.428 52.959) (width 0.254) (layer B.Cu) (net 8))
 (segment (start 114.935 55.245) (end 114.935 56.10098) (width 0.254) (layer B.Cu) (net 8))
 (segment (start 122.9106 53.4416) (end 122.428 52.959) (width 0.254) (layer B.Cu) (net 8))
 (segment (start 130.175 60.0075) (end 130.175 58.19902) (width 0.254) (layer B.Cu) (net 13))
 (segment (start 128.524 53.594) (end 128.397 53.594) (width 0.254) (layer F.Cu) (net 9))
 (segment (start 128.397 53.594) (end 127.5715 52.7685) (width 0.254) (layer F.Cu) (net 9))
 (segment (start 122.2502 54.1782) (end 122.2502 55.626) (width 0.254) (layer B.Cu) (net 9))
 (segment (start 122.047 53.975) (end 122.2502 54.1782) (width 0.254) (layer B.Cu) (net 9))
 (via (at 122.047 53.975) (size 0.8) (drill 0.5) (layers F.Cu B.Cu) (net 9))
 (segment (start 122.174 53.848) (end 122.047 53.975) (width 0.254) (layer F.Cu) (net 9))
 (segment (start 122.174 53.34) (end 122.174 53.848) (width 0.254) (layer F.Cu) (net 9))
 (segment (start 122.7455 52.7685) (end 122.174 53.34) (width 0.254) (layer F.Cu) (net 9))
 (segment (start 127.5715 52.7685) (end 122.7455 52.7685) (width 0.254) (layer F.Cu) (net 9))
 (segment (start 130.175 56.10098) (end 130.175 54.102) (width 0.254) (layer B.Cu) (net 9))
 (segment (start 129.667 53.594) (end 128.524 53.594) (width 0.254) (layer F.Cu) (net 9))
 (segment (start 130.048 53.975) (end 129.667 53.594) (width 0.254) (layer F.Cu) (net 9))
 (via (at 130.048 53.975) (size 0.8) (drill 0.5) (layers F.Cu B.Cu) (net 9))
 (segment (start 130.175 54.102) (end 130.048 53.975) (width 0.254) (layer B.Cu) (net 9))
 (segment (start 117.7925 58.42) (end 115.15598 58.42) (width 0.254) (layer B.Cu) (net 14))
 (segment (start 115.15598 58.42) (end 114.935 58.19902) (width 0.254) (layer B.Cu) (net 14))
 (segment (start 121.06402 60.96) (end 121.06402 58.95848) (width 0.254) (layer B.Cu) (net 15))
 (segment (start 121.06402 58.95848) (end 121.6025 58.42) (width 0.254) (layer B.Cu) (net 15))
 (segment (start 127.3175 58.42) (end 127.3175 57.57926) (width 0.254) (layer B.Cu) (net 2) (status 400000))
 (segment (start 130.08176 46.15) (end 111.555 46.15) (width 0.254) (layer F.Cu) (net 2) (status 800000))
 (segment (start 131.65328 47.72152) (end 130.08176 46.15) (width 0.254) (layer F.Cu) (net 2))
 (segment (start 131.65328 54.40172) (end 131.65328 47.72152) (width 0.254) (layer F.Cu) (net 2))
 (segment (start 130.90144 55.15356) (end 131.65328 54.40172) (width 0.254) (layer F.Cu) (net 2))
 (segment (start 130.07848 55.15356) (end 130.90144 55.15356) (width 0.254) (layer F.Cu) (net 2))
 (segment (start 129.2606 54.33568) (end 130.07848 55.15356) (width 0.254) (layer F.Cu) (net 2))
 (segment (start 128.69164 54.33568) (end 129.2606 54.33568) (width 0.254) (layer F.Cu) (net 2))
 (segment (start 128.12268 54.90464) (end 128.69164 54.33568) (width 0.254) (layer F.Cu) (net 2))
 (segment (start 128.12268 56.77408) (end 128.12268 54.90464) (width 0.254) (layer F.Cu) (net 2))
 (segment (start 128.05156 56.8452) (end 128.12268 56.77408) (width 0.254) (layer F.Cu) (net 2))
 (via (at 128.05156 56.8452) (size 0.889) (layers F.Cu B.Cu) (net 2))
 (segment (start 127.3175 57.57926) (end 128.05156 56.8452) (width 0.254) (layer B.Cu) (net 2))
 (segment (start 114.9985 62.23) (end 114.554 62.23) (width 0.254) (layer F.Cu) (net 2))
 (segment (start 113.1697 63.6143) (end 113.1697 64.6176) (width 0.254) (layer F.Cu) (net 2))
 (segment (start 114.554 62.23) (end 113.1697 63.6143) (width 0.254) (layer F.Cu) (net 2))
 (segment (start 120.9548 48.514) (end 120.9548 46.7614) (width 0.254) (layer B.Cu) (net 2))
 (segment (start 120.9548 46.7614) (end 120.3434 46.15) (width 0.254) (layer B.Cu) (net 2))
 (segment (start 120.3434 46.15) (end 111.555 46.15) (width 0.254) (layer B.Cu) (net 2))
 (segment (start 113.411 63.754) (end 113.4745 63.754) (width 0.254) (layer B.Cu) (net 2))
 (segment (start 112.776 47.371) (end 111.555 46.15) (width 0.254) (layer F.Cu) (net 2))
 (segment (start 114.9985 62.23) (end 112.776 60.0075) (width 0.254) (layer F.Cu) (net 2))
 (segment (start 112.776 60.0075) (end 112.776 47.371) (width 0.254) (layer F.Cu) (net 2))
 (via (at 114.9985 62.23) (size 0.889) (layers F.Cu B.Cu) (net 2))
 (segment (start 113.4745 63.754) (end 114.9985 62.23) (width 0.254) (layer B.Cu) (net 2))
 (segment (start 126.1872 55.626) (end 126.1872 56.9722) (width 0.254) (layer B.Cu) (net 2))
 (segment (start 127.3175 58.1025) (end 126.365 57.15) (width 0.254) (layer B.Cu) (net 2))
 (segment (start 127.3175 58.1025) (end 127.3175 58.42) (width 0.254) (layer B.Cu) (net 2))
 (segment (start 126.1872 56.9722) (end 126.365 57.15) (width 0.254) (layer B.Cu) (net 2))
 (segment (start 115.8875 50.165) (end 116.84 50.165) (width 0.254) (layer B.Cu) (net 1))
 (segment (start 118.491 48.514) (end 118.999 48.514) (width 0.254) (layer B.Cu) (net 1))
 (segment (start 116.84 50.165) (end 118.491 48.514) (width 0.254) (layer B.Cu) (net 1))
 (segment (start 115.8621 70.9803) (end 115.3795 70.9803) (width 0.254) (layer F.Cu) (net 7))
 (segment (start 114.9985 70.5993) (end 114.9985 69.2404) (width 0.254) (layer F.Cu) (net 7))
 (segment (start 115.3795 70.9803) (end 114.9985 70.5993) (width 0.254) (layer F.Cu) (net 7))
 (segment (start 123.5075 58.42) (end 123.5075 57.4675) (width 0.254) (layer B.Cu) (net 7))
 (via (at 123.5075 57.4675) (size 0.889) (layers F.Cu B.Cu) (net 7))
 (segment (start 123.4948 57.4802) (end 123.4948 58.3946) (width 0.254) (layer F.Cu) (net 7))
 (segment (start 123.5075 57.4675) (end 123.4948 57.4802) (width 0.254) (layer F.Cu) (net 7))
 (segment (start 130.175 61.9125) (end 130.175 70.612) (width 0.5) (layer B.Cu) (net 7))
 (segment (start 115.951 62.8269) (end 115.951 63.754) (width 0.5) (layer B.Cu) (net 7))
 (segment (start 116.0653 62.7126) (end 115.951 62.8269) (width 0.5) (layer B.Cu) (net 7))
 (via (at 116.0653 62.7126) (size 0.889) (layers F.Cu B.Cu) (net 7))
 (segment (start 116.0653 70.7771) (end 116.0653 62.7126) (width 0.5) (layer F.Cu) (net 7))
 (segment (start 115.8621 70.9803) (end 116.0653 70.7771) (width 0.5) (layer F.Cu) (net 7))
 (via (at 115.8621 70.9803) (size 0.889) (layers F.Cu B.Cu) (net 7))
 (segment (start 115.8621 71.1708) (end 115.8621 70.9803) (width 0.5) (layer B.Cu) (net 7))
 (segment (start 116.4717 71.7804) (end 115.8621 71.1708) (width 0.5) (layer B.Cu) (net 7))
 (segment (start 129.0066 71.7804) (end 116.4717 71.7804) (width 0.5) (layer B.Cu) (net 7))
 (segment (start 130.175 70.612) (end 129.0066 71.7804) (width 0.5) (layer B.Cu) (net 7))
 (segment (start 124.841 52.959) (end 124.841 54.737) (width 0.5) (layer B.Cu) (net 7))
 (segment (start 129.54 50.4825) (end 127.3175 50.4825) (width 0.5) (layer B.Cu) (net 7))
 (segment (start 127.3175 50.4825) (end 124.841 52.959) (width 0.5) (layer B.Cu) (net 7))
 (segment (start 130.175 61.9125) (end 131.3815 61.9125) (width 0.5) (layer B.Cu) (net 7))
 (segment (start 131.572 52.5145) (end 129.54 50.4825) (width 0.5) (layer B.Cu) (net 7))
 (segment (start 131.572 61.722) (end 131.572 52.5145) (width 0.5) (layer B.Cu) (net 7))
 (segment (start 131.3815 61.9125) (end 131.572 61.722) (width 0.5) (layer B.Cu) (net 7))
 (segment (start 124.841 55.626) (end 124.841 54.737) (width 0.254) (layer B.Cu) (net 7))
 (segment (start 119.6975 58.42) (end 119.6975 57.4675) (width 0.254) (layer B.Cu) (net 7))
 (segment (start 123.19 57.15) (end 123.5075 57.4675) (width 0.254) (layer B.Cu) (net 7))
 (segment (start 120.015 57.15) (end 123.19 57.15) (width 0.254) (layer B.Cu) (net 7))
 (segment (start 119.6975 57.4675) (end 120.015 57.15) (width 0.254) (layer B.Cu) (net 7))
 (segment (start 126.746 60.96) (end 127 60.96) (width 0.5) (layer B.Cu) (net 7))
 (segment (start 127.9525 61.9125) (end 130.175 61.9125) (width 0.5) (layer B.Cu) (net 7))
 (segment (start 127 60.96) (end 127.9525 61.9125) (width 0.5) (layer B.Cu) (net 7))
 (segment (start 124.206 55.626) (end 124.206 57.7215) (width 0.254) (layer B.Cu) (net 7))
 (segment (start 124.206 57.7215) (end 123.5075 58.42) (width 0.254) (layer B.Cu) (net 7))
 (segment (start 124.206 55.626) (end 124.841 55.626) (width 0.254) (layer B.Cu) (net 7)))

